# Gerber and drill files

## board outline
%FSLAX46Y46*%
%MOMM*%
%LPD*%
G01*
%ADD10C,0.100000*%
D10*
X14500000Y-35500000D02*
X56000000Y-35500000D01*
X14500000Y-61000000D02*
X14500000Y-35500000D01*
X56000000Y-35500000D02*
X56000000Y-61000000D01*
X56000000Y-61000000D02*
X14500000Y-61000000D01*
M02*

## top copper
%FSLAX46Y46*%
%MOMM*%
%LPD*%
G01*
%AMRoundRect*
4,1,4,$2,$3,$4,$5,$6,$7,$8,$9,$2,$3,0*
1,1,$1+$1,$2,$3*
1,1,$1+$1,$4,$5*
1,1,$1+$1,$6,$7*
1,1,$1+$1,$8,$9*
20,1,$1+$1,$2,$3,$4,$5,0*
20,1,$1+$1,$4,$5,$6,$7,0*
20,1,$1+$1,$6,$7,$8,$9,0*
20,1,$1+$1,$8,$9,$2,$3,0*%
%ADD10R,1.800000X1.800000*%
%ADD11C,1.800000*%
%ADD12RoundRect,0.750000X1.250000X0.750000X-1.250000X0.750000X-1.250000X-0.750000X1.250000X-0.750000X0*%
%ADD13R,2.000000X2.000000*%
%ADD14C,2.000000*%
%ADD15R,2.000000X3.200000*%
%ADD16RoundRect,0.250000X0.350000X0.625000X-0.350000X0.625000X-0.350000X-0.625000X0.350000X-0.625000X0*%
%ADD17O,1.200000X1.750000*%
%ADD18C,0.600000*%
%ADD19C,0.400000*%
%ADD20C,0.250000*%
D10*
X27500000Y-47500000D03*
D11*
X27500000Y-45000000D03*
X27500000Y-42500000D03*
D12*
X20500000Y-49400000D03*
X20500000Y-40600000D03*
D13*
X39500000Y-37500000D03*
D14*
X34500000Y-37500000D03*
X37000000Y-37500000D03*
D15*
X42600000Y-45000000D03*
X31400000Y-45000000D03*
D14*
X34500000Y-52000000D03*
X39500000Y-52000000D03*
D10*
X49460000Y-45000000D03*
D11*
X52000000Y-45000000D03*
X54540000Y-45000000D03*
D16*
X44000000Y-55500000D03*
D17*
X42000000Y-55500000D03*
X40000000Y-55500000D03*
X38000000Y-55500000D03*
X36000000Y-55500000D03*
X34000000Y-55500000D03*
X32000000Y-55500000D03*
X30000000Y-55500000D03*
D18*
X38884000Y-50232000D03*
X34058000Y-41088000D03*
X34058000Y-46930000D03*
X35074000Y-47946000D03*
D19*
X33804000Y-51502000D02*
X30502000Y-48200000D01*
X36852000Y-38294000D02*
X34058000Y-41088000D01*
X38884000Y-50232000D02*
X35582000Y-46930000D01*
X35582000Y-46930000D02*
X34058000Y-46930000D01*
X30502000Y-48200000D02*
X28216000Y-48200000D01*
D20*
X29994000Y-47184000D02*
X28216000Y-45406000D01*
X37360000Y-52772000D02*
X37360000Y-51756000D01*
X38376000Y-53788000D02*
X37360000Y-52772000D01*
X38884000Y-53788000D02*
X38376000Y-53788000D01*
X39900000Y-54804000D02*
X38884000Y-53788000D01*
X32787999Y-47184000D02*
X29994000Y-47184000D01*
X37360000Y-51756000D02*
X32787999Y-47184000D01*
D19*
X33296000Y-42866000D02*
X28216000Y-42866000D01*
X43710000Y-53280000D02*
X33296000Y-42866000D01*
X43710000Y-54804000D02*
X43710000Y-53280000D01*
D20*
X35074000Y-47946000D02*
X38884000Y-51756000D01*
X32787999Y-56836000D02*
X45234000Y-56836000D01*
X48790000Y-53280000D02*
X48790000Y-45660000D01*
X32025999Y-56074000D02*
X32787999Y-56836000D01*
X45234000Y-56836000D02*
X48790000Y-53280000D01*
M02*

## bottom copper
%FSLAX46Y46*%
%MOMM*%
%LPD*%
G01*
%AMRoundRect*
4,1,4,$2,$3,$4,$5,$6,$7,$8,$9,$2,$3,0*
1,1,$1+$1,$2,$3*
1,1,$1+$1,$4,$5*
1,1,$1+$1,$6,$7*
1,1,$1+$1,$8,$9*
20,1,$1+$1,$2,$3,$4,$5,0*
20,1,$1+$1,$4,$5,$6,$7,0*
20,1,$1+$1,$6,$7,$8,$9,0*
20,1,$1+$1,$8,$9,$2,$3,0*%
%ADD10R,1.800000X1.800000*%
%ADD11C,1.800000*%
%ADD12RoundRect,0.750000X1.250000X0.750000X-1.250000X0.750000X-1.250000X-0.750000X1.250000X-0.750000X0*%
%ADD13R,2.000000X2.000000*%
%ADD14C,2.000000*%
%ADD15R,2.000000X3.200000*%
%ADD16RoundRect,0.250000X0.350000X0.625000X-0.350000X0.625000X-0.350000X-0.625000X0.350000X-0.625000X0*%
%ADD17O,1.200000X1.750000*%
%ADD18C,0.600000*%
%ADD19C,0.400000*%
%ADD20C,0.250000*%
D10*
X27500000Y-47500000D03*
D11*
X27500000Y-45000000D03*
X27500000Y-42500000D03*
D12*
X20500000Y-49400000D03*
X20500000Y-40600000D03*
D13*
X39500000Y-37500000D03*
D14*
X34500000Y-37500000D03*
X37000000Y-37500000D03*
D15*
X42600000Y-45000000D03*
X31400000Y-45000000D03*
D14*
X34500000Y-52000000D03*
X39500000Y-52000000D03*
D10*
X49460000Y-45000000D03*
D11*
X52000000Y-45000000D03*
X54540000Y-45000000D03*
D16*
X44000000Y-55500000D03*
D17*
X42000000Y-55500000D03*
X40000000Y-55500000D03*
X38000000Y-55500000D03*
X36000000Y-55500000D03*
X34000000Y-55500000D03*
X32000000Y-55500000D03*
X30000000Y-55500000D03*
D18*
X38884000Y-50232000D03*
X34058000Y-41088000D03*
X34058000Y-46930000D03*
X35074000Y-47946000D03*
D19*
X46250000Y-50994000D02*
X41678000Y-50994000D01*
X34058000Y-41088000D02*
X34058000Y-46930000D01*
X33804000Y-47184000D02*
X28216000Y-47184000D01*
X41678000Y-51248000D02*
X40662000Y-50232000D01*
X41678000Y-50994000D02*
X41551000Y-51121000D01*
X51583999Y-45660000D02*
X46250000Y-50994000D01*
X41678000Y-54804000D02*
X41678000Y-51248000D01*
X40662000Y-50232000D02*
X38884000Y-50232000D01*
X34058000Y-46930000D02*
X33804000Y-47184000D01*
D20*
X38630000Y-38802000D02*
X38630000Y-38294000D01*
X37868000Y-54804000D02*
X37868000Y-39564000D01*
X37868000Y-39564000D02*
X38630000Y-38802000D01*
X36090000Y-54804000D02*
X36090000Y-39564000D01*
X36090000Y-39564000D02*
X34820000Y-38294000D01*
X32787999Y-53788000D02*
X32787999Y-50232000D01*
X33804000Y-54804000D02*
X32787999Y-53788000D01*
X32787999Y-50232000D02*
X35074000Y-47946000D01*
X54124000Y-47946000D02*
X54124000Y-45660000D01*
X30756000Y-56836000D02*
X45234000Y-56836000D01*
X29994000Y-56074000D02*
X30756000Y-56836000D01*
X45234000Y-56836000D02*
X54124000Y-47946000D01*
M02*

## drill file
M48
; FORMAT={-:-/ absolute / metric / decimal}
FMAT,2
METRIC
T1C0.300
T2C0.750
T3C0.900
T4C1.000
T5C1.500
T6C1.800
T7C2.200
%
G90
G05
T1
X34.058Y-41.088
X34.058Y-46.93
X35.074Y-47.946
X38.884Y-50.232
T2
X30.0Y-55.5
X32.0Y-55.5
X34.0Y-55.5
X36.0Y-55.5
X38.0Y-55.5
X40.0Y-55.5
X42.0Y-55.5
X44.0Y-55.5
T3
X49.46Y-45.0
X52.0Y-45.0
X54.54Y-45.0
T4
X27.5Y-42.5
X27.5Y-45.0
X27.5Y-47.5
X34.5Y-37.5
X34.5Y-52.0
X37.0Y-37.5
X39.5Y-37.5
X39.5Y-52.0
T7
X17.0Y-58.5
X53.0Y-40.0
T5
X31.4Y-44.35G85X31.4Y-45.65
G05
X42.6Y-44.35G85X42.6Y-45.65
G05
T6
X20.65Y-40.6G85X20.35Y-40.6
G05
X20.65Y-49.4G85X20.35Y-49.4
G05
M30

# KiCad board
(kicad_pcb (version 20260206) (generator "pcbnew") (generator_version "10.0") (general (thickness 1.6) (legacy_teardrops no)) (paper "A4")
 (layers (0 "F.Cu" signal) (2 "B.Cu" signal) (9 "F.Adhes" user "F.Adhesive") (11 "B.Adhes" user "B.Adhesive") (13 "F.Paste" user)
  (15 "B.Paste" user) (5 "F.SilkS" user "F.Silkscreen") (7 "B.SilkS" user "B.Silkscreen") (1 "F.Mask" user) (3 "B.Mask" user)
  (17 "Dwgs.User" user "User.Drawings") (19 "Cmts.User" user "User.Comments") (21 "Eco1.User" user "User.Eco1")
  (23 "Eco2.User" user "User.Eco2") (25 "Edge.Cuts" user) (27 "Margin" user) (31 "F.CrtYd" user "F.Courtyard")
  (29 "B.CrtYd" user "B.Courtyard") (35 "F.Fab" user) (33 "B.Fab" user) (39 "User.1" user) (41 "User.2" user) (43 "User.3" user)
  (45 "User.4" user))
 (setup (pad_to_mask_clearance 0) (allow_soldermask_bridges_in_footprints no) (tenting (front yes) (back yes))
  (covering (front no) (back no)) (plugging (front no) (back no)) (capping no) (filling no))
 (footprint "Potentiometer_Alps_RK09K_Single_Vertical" (layer "F.Cu") (at 27.5 47.5 180)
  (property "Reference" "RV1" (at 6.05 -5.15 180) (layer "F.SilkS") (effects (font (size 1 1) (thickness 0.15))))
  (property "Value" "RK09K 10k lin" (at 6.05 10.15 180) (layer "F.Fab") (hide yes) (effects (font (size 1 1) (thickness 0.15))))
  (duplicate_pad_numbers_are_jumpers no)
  (pad "1" thru_hole rect (at 0 0 180) (size 1.8 1.8) (drill 1) (layers "*.Cu" "*.Mask") (remove_unused_layers no) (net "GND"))
  (pad "2" thru_hole circle (at 0 2.5 180) (size 1.8 1.8) (drill 1) (layers "*.Cu" "*.Mask") (remove_unused_layers no) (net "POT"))
  (pad "3" thru_hole circle (at 0 5 180) (size 1.8 1.8) (drill 1) (layers "*.Cu" "*.Mask") (remove_unused_layers no) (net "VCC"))
  (pad "MP" thru_hole roundrect (at 7 -1.9 180) (size 4 3) (drill oval 2.1 1.8) (layers "*.Cu" "*.Mask") (remove_unused_layers no)
   (roundrect_rratio 0.25))
  (pad "MP" thru_hole roundrect (at 7 6.9 180) (size 4 3) (drill oval 2.1 1.8) (layers "*.Cu" "*.Mask") (remove_unused_layers no)
   (roundrect_rratio 0.25)))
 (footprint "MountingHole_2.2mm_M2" (layer "F.Cu") (at 53 40)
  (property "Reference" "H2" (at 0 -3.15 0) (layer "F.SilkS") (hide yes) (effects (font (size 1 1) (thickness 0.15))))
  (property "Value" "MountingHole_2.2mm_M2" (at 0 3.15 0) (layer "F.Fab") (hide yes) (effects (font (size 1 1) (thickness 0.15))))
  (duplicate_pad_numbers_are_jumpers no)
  (pad "" np_thru_hole circle (at 0 0) (size 2.2 2.2) (drill 2.2) (layers "*.Cu" "*.Mask")))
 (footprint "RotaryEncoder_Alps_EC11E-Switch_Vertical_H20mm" (layer "F.Cu") (at 39.5 37.5 -90)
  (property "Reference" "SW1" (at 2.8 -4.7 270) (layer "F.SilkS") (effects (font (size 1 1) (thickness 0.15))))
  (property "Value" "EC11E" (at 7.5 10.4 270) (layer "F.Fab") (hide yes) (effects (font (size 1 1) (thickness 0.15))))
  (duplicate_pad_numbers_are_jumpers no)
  (pad "A" thru_hole rect (at 0 0 270) (size 2 2) (drill 1) (layers "*.Cu" "*.Mask") (remove_unused_layers no) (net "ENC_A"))
  (pad "B" thru_hole circle (at 0 5 270) (size 2 2) (drill 1) (layers "*.Cu" "*.Mask") (remove_unused_layers no) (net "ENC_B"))
  (pad "C" thru_hole circle (at 0 2.5 270) (size 2 2) (drill 1) (layers "*.Cu" "*.Mask") (remove_unused_layers no) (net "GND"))
  (pad "MP" thru_hole rect (at 7.5 -3.1 270) (size 3.2 2) (drill oval 2.8 1.5) (layers "*.Cu" "*.Mask") (remove_unused_layers no))
  (pad "MP" thru_hole rect (at 7.5 8.1 270) (size 3.2 2) (drill oval 2.8 1.5) (layers "*.Cu" "*.Mask") (remove_unused_layers no))
  (pad "S1" thru_hole circle (at 14.5 5 270) (size 2 2) (drill 1) (layers "*.Cu" "*.Mask") (remove_unused_layers no) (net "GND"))
  (pad "S2" thru_hole circle (at 14.5 0 270) (size 2 2) (drill 1) (layers "*.Cu" "*.Mask") (remove_unused_layers no) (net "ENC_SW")))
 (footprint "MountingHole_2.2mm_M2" (layer "F.Cu") (at 17 58.5)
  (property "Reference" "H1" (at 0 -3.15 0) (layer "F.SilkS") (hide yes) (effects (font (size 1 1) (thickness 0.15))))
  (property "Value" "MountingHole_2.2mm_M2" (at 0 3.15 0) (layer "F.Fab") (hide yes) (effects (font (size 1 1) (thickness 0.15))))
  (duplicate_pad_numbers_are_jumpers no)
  (pad "" np_thru_hole circle (at 0 0) (size 2.2 2.2) (drill 2.2) (layers "*.Cu" "*.Mask")))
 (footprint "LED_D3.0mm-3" (layer "F.Cu") (at 49.46 45)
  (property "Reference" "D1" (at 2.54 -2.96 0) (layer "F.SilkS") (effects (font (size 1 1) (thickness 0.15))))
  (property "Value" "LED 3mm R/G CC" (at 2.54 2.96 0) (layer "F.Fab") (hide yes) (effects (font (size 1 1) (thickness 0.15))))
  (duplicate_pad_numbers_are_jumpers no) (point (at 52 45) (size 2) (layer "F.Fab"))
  (pad "1" thru_hole rect (at 0 0) (size 1.8 1.8) (drill 0.9) (layers "*.Cu" "*.Mask") (remove_unused_layers no) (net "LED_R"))
  (pad "2" thru_hole circle (at 2.54 0) (size 1.8 1.8) (drill 0.9) (layers "*.Cu" "*.Mask") (remove_unused_layers no) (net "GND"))
  (pad "3" thru_hole circle (at 5.08 0) (size 1.8 1.8) (drill 0.9) (layers "*.Cu" "*.Mask") (remove_unused_layers no) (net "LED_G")))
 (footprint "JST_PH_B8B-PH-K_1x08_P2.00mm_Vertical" (layer "B.Cu") (at 44 55.5 180)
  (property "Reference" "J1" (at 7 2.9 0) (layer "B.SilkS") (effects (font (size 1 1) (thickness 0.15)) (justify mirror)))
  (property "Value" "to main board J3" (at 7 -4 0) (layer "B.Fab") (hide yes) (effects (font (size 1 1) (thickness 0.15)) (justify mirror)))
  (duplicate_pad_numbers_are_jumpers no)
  (pad "1" thru_hole roundrect (at 0 0 180) (size 1.2 1.75) (drill 0.75) (layers "*.Cu" "*.Mask") (remove_unused_layers no)
   (roundrect_rratio 0.208333) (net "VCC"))
  (pad "2" thru_hole oval (at 2 0 180) (size 1.2 1.75) (drill 0.75) (layers "*.Cu" "*.Mask") (remove_unused_layers no) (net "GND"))
  (pad "3" thru_hole oval (at 4 0 180) (size 1.2 1.75) (drill 0.75) (layers "*.Cu" "*.Mask") (remove_unused_layers no) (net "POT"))
  (pad "4" thru_hole oval (at 6 0 180) (size 1.2 1.75) (drill 0.75) (layers "*.Cu" "*.Mask") (remove_unused_layers no) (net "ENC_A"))
  (pad "5" thru_hole oval (at 8 0 180) (size 1.2 1.75) (drill 0.75) (layers "*.Cu" "*.Mask") (remove_unused_layers no) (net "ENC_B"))
  (pad "6" thru_hole oval (at 10 0 180) (size 1.2 1.75) (drill 0.75) (layers "*.Cu" "*.Mask") (remove_unused_layers no) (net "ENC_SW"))
  (pad "7" thru_hole oval (at 12 0 180) (size 1.2 1.75) (drill 0.75) (layers "*.Cu" "*.Mask") (remove_unused_layers no) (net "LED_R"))
  (pad "8" thru_hole oval (at 14 0 180) (size 1.2 1.75) (drill 0.75) (layers "*.Cu" "*.Mask") (remove_unused_layers no) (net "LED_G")))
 (gr_line (start 14.5 35.5) (end 56 35.5) (stroke (width 0.1) (type default)) (layer "Edge.Cuts"))
 (gr_line (start 14.5 61) (end 14.5 35.5) (stroke (width 0.1) (type default)) (layer "Edge.Cuts"))
 (gr_line (start 56 35.5) (end 56 61) (stroke (width 0.1) (type default)) (layer "Edge.Cuts"))
 (gr_line (start 56 61) (end 14.5 61) (stroke (width 0.1) (type default)) (layer "Edge.Cuts"))
 (segment (start 33.804 51.502) (end 30.502 48.2) (width 0.4) (layer "F.Cu") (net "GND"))
 (segment (start 36.852 38.294) (end 34.058 41.088) (width 0.4) (layer "F.Cu") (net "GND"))
 (segment (start 38.884 50.232) (end 35.582 46.93) (width 0.4) (layer "F.Cu") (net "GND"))
 (segment (start 35.582 46.93) (end 34.058 46.93) (width 0.4) (layer "F.Cu") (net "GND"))
 (segment (start 30.502 48.2) (end 28.216 48.2) (width 0.4) (layer "F.Cu") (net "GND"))
 (via (at 38.884 50.232) (size 0.6) (drill 0.3) (layers "F.Cu" "B.Cu") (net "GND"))
 (via (at 34.058 41.088) (size 0.6) (drill 0.3) (layers "F.Cu" "B.Cu") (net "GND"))
 (via (at 34.058 46.93) (size 0.6) (drill 0.3) (layers "F.Cu" "B.Cu") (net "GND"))
 (segment (start 46.25 50.994) (end 41.678 50.994) (width 0.4) (layer "B.Cu") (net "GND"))
 (segment (start 34.058 41.088) (end 34.058 46.93) (width 0.4) (layer "B.Cu") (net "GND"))
 (segment (start 33.804 47.184) (end 28.216 47.184) (width 0.4) (layer "B.Cu") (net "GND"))
 (segment (start 41.678 51.248) (end 40.662 50.232) (width 0.4) (layer "B.Cu") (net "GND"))
 (segment (start 41.678 50.994) (end 41.551 51.121) (width 0.4) (layer "B.Cu") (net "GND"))
 (segment (start 51.583999 45.66) (end 46.25 50.994) (width 0.4) (layer "B.Cu") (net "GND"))
 (segment (start 41.678 54.804) (end 41.678 51.248) (width 0.4) (layer "B.Cu") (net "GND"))
 (segment (start 40.662 50.232) (end 38.884 50.232) (width 0.4) (layer "B.Cu") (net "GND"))
 (segment (start 34.058 46.93) (end 33.804 47.184) (width 0.4) (layer "B.Cu") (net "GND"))
 (segment (start 29.994 47.184) (end 28.216 45.406) (width 0.25) (layer "F.Cu") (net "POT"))
 (segment (start 37.36 52.772) (end 37.36 51.756) (width 0.25) (layer "F.Cu") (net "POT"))
 (segment (start 38.376 53.788) (end 37.36 52.772) (width 0.25) (layer "F.Cu") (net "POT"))
 (segment (start 38.884 53.788) (end 38.376 53.788) (width 0.25) (layer "F.Cu") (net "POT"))
 (segment (start 39.9 54.804) (end 38.884 53.788) (width 0.25) (layer "F.Cu") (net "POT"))
 (segment (start 32.787999 47.184) (end 29.994 47.184) (width 0.25) (layer "F.Cu") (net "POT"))
 (segment (start 37.36 51.756) (end 32.787999 47.184) (width 0.25) (layer "F.Cu") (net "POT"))
 (segment (start 33.296 42.866) (end 28.216 42.866) (width 0.4) (layer "F.Cu") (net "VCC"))
 (segment (start 43.71 53.28) (end 33.296 42.866) (width 0.4) (layer "F.Cu") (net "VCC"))
 (segment (start 43.71 54.804) (end 43.71 53.28) (width 0.4) (layer "F.Cu") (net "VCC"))
 (segment (start 38.63 38.802) (end 38.63 38.294) (width 0.25) (layer "B.Cu") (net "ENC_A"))
 (segment (start 37.868 54.804) (end 37.868 39.564) (width 0.25) (layer "B.Cu") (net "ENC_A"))
 (segment (start 37.868 39.564) (end 38.63 38.802) (width 0.25) (layer "B.Cu") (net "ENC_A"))
 (segment (start 36.09 54.804) (end 36.09 39.564) (width 0.25) (layer "B.Cu") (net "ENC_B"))
 (segment (start 36.09 39.564) (end 34.82 38.294) (width 0.25) (layer "B.Cu") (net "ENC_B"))
 (segment (start 35.074 47.946) (end 38.884 51.756) (width 0.25) (layer "F.Cu") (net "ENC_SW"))
 (via (at 35.074 47.946) (size 0.6) (drill 0.3) (layers "F.Cu" "B.Cu") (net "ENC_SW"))
 (segment (start 32.787999 53.788) (end 32.787999 50.232) (width 0.25) (layer "B.Cu") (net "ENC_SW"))
 (segment (start 33.804 54.804) (end 32.787999 53.788) (width 0.25) (layer "B.Cu") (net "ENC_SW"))
 (segment (start 32.787999 50.232) (end 35.074 47.946) (width 0.25) (layer "B.Cu") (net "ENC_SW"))
 (segment (start 32.787999 56.836) (end 45.234 56.836) (width 0.25) (layer "F.Cu") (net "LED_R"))
 (segment (start 48.79 53.28) (end 48.79 45.66) (width 0.25) (layer "F.Cu") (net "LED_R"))
 (segment (start 32.025999 56.074) (end 32.787999 56.836) (width 0.25) (layer "F.Cu") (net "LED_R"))
 (segment (start 45.234 56.836) (end 48.79 53.28) (width 0.25) (layer "F.Cu") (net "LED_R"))
 (segment (start 54.124 47.946) (end 54.124 45.66) (width 0.25) (layer "B.Cu") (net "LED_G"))
 (segment (start 30.756 56.836) (end 45.234 56.836) (width 0.25) (layer "B.Cu") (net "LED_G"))
 (segment (start 29.994 56.074) (end 30.756 56.836) (width 0.25) (layer "B.Cu") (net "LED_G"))
 (segment (start 45.234 56.836) (end 54.124 47.946) (width 0.25) (layer "B.Cu") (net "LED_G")))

